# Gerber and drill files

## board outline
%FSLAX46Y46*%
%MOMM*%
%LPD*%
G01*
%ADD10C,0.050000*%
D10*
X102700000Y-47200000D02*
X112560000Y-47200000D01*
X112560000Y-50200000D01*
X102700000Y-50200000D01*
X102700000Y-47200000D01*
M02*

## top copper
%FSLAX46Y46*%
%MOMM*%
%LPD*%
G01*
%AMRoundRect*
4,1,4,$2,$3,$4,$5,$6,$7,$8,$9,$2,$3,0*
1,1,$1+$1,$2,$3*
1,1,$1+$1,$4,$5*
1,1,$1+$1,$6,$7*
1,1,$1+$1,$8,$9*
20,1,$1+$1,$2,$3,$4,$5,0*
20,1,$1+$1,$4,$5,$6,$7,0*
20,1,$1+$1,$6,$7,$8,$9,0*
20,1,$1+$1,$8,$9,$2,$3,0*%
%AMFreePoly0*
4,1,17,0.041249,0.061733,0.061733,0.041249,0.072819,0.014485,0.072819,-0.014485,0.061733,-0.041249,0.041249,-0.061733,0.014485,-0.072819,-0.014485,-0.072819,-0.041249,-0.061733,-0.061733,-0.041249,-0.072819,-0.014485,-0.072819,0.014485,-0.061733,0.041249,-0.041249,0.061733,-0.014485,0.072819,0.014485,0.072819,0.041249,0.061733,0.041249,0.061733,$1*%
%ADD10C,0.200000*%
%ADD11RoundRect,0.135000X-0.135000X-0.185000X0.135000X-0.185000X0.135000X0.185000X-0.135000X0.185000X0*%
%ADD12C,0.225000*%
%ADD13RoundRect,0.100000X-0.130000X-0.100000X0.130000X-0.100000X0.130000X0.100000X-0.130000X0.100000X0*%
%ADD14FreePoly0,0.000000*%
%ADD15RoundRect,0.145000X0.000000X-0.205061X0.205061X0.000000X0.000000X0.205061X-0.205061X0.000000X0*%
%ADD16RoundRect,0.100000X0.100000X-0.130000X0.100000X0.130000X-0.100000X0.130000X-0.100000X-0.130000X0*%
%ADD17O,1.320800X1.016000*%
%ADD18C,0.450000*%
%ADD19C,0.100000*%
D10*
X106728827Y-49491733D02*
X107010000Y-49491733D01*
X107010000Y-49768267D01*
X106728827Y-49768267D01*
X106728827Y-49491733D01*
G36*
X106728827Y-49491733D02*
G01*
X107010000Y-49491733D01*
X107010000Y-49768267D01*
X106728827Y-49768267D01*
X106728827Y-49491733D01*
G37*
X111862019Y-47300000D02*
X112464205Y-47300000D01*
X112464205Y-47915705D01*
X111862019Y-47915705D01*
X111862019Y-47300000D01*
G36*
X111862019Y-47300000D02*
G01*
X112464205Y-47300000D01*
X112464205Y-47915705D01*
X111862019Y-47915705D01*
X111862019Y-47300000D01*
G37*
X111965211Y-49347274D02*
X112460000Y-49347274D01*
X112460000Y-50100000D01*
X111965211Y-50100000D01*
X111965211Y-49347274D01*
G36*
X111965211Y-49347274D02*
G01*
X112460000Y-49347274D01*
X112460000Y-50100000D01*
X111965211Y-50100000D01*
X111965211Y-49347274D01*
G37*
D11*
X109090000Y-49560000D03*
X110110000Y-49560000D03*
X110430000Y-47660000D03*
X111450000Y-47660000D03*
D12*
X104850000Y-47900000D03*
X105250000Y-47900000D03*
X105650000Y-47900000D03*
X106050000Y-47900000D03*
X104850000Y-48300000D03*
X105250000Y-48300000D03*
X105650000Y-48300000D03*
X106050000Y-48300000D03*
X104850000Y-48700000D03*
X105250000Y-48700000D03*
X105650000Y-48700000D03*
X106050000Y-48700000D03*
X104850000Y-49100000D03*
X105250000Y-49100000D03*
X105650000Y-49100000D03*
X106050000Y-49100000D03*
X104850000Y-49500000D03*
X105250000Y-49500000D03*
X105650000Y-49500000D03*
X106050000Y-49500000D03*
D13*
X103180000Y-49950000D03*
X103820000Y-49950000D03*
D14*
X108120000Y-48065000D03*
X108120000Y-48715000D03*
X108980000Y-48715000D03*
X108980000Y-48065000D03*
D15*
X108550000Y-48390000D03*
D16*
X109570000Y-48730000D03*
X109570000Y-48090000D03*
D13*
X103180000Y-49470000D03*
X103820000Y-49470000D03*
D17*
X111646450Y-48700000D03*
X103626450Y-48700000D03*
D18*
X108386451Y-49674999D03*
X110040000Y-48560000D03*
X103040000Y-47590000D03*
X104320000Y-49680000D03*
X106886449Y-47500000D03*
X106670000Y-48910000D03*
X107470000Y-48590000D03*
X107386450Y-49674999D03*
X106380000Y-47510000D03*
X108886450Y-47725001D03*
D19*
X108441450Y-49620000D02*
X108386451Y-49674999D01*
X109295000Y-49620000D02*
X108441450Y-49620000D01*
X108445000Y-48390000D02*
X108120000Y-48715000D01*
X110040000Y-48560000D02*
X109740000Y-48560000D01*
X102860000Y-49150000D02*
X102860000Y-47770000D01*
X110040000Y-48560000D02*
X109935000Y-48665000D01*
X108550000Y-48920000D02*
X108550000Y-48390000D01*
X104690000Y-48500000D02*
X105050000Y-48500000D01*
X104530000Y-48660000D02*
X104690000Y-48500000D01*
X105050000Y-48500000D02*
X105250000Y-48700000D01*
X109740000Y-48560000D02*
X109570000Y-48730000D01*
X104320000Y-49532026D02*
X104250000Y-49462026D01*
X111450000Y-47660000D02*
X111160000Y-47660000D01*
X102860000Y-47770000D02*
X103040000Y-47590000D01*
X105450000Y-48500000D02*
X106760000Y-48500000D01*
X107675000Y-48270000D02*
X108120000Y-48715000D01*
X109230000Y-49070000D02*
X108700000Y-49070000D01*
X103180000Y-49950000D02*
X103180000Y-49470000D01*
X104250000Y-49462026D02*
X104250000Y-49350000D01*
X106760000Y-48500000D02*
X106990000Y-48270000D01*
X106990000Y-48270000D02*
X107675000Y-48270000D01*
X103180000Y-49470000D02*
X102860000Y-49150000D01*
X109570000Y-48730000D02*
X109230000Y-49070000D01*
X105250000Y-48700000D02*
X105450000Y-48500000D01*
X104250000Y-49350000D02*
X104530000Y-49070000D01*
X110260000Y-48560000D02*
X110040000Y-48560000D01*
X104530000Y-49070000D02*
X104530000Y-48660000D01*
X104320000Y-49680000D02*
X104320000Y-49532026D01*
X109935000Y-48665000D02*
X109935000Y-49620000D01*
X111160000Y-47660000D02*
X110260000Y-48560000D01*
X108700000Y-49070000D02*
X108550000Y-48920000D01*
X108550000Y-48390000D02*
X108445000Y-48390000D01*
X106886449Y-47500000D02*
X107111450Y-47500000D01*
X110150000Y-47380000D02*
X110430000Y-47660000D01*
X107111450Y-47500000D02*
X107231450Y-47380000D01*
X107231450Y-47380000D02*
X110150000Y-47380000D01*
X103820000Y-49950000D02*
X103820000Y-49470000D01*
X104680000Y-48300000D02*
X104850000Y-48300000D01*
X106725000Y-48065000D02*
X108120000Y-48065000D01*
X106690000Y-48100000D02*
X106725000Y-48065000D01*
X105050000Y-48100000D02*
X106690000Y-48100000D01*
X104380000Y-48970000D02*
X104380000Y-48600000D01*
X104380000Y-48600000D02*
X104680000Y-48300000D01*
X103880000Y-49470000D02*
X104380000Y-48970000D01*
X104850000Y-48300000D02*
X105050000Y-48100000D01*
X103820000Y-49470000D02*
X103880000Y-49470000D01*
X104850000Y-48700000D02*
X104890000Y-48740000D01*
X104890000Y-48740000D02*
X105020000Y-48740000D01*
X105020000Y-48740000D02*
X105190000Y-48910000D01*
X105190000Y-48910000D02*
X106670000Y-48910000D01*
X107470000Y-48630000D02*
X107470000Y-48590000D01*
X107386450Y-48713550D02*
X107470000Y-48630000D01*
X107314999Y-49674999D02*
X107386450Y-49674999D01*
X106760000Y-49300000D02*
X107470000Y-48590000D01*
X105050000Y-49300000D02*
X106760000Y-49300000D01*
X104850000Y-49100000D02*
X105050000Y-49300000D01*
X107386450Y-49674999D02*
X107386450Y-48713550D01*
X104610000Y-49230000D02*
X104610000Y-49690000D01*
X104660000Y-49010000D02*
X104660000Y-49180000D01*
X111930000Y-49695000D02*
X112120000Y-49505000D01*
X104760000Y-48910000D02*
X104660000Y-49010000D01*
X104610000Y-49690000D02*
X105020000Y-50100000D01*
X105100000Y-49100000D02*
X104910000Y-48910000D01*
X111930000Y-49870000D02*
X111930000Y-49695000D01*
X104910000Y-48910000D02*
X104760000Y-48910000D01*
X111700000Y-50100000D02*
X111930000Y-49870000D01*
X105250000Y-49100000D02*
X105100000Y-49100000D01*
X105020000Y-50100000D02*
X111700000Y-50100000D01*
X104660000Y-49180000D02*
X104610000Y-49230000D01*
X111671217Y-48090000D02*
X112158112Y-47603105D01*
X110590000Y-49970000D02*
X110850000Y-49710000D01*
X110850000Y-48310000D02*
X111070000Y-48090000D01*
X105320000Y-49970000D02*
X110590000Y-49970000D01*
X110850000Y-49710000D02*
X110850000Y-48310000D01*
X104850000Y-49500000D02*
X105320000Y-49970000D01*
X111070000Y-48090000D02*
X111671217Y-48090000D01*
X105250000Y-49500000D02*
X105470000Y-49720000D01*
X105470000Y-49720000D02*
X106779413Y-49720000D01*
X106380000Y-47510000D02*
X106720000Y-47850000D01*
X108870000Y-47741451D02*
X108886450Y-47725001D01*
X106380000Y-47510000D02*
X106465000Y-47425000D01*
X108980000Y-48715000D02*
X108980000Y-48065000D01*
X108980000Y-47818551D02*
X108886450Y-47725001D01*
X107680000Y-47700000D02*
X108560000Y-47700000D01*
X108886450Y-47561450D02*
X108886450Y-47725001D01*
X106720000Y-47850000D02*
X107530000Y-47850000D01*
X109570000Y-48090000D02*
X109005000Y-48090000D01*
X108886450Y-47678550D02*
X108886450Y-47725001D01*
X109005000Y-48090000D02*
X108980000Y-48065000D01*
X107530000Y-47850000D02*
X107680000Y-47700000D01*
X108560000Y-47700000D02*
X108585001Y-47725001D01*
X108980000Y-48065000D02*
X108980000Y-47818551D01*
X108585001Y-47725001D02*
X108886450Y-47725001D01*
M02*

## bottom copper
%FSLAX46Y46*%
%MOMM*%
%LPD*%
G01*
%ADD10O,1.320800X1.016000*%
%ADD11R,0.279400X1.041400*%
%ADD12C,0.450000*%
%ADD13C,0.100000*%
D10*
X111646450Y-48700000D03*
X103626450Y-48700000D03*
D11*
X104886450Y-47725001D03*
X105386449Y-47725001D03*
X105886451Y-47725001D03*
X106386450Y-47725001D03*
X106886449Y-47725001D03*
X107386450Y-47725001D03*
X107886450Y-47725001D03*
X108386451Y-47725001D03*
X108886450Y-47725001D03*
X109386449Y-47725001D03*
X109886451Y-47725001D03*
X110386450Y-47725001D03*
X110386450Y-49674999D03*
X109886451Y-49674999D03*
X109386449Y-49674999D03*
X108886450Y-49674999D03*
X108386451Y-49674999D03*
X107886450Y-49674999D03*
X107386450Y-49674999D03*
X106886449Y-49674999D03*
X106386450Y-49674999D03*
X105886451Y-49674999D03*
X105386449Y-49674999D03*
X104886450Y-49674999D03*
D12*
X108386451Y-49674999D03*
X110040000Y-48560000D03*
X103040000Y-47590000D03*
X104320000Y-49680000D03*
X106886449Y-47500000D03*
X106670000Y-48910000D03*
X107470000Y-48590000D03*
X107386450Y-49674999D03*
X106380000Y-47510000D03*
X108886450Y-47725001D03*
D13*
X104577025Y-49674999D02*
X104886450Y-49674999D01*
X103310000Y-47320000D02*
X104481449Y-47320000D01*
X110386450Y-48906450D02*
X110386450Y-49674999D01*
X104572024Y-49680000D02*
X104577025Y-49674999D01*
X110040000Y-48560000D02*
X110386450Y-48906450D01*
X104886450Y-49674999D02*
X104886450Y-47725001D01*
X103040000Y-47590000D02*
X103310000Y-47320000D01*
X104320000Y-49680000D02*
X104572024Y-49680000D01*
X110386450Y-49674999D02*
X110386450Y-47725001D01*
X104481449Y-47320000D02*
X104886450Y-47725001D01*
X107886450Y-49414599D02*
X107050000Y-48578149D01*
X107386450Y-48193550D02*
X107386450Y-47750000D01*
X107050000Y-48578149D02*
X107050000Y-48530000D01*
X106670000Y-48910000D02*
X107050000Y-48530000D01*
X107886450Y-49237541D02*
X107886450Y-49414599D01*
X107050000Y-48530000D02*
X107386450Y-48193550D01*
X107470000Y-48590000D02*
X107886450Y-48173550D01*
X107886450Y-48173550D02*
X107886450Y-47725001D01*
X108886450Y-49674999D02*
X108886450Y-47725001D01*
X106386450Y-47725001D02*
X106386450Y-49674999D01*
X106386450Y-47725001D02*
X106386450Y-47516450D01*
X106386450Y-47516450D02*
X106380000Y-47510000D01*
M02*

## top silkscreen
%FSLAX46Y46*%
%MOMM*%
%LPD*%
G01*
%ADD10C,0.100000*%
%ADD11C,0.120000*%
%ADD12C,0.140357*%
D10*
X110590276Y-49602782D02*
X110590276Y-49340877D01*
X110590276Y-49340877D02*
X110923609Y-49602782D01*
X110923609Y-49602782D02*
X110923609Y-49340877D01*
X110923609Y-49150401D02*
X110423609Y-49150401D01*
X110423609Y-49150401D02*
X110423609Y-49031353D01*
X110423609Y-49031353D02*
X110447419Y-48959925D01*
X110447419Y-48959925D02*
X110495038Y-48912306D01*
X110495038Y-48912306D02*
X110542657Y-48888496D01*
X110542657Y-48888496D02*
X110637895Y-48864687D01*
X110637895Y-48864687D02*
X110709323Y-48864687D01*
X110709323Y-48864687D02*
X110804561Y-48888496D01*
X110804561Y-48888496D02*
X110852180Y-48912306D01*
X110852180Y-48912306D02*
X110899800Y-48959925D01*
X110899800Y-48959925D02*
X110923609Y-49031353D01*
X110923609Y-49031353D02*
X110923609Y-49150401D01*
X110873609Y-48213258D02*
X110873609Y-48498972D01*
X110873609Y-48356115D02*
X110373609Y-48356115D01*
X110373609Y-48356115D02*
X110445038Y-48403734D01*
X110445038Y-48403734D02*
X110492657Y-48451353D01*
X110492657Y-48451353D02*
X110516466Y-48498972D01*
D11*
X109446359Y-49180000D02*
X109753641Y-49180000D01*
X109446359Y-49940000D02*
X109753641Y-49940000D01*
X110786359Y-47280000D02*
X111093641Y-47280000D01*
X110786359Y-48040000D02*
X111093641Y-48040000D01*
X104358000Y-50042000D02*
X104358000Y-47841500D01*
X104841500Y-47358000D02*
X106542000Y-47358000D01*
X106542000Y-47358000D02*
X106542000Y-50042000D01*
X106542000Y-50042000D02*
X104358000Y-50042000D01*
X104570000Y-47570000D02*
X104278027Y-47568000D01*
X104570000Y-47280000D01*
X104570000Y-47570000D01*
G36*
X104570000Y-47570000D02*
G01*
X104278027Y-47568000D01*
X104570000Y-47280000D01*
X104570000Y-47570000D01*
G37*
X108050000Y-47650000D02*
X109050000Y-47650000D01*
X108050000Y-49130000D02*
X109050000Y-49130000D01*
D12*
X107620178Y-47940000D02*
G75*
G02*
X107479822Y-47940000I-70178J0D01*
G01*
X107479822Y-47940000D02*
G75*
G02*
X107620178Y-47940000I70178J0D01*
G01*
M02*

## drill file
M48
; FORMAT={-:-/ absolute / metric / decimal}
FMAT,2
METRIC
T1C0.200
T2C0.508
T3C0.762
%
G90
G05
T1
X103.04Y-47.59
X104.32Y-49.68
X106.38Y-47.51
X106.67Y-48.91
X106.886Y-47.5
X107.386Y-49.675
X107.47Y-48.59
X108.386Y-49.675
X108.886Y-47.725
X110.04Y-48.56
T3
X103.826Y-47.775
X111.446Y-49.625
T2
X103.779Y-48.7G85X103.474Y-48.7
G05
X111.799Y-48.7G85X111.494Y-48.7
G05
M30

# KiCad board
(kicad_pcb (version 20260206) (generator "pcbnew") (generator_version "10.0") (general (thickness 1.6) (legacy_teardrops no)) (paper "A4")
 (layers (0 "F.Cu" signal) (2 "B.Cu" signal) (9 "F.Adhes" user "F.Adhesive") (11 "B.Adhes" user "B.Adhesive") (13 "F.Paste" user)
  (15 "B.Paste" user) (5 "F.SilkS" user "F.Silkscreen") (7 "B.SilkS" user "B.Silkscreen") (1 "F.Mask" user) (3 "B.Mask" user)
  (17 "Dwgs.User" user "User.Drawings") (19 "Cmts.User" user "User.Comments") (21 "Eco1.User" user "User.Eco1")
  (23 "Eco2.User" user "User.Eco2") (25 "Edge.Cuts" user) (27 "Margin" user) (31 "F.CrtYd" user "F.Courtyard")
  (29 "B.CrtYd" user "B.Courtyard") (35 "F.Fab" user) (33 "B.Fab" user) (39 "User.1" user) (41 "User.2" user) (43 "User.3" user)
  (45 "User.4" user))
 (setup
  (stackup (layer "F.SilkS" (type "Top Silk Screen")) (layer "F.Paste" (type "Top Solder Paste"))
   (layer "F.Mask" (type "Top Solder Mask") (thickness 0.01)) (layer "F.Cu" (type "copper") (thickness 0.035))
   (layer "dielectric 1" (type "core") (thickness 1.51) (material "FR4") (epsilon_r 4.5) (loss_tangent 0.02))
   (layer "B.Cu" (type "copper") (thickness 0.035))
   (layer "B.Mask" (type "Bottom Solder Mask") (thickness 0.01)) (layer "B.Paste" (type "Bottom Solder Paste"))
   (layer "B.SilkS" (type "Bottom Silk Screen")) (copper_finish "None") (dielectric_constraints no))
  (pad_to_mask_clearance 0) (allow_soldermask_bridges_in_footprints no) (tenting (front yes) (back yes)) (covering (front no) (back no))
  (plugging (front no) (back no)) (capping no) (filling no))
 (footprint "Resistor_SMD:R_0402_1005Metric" (layer "F.Cu") (at 109.6 49.56)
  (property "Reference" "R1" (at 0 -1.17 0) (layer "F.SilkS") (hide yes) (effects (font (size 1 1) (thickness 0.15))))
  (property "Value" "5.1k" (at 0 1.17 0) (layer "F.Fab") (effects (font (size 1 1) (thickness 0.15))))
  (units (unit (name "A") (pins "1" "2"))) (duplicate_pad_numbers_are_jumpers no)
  (fp_line (start -0.153641 -0.38) (end 0.153641 -0.38) (stroke (width 0.12) (type solid)) (layer "F.SilkS"))
  (fp_line (start -0.153641 0.38) (end 0.153641 0.38) (stroke (width 0.12) (type solid)) (layer "F.SilkS"))
  (pad "1" smd roundrect (at -0.51 0) (size 0.54 0.64) (layers "F.Cu" "F.Mask" "F.Paste") (roundrect_rratio 0.25) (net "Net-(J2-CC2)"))
  (pad "2" smd roundrect (at 0.51 0) (size 0.54 0.64) (layers "F.Cu" "F.Mask" "F.Paste") (roundrect_rratio 0.25) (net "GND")))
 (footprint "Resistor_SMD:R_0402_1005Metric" (layer "F.Cu") (at 110.94 47.66)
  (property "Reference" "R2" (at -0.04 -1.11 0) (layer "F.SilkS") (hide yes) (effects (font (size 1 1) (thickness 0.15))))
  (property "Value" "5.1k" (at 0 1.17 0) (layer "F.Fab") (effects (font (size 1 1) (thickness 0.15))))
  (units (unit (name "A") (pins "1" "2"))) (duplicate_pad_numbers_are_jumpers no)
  (fp_line (start -0.153641 -0.38) (end 0.153641 -0.38) (stroke (width 0.12) (type solid)) (layer "F.SilkS"))
  (fp_line (start -0.153641 0.38) (end 0.153641 0.38) (stroke (width 0.12) (type solid)) (layer "F.SilkS"))
  (pad "1" smd roundrect (at -0.51 0) (size 0.54 0.64) (layers "F.Cu" "F.Mask" "F.Paste") (roundrect_rratio 0.25) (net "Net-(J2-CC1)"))
  (pad "2" smd roundrect (at 0.51 0) (size 0.54 0.64) (layers "F.Cu" "F.Mask" "F.Paste") (roundrect_rratio 0.25) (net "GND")))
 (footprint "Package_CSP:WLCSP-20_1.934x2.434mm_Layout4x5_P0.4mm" (layer "F.Cu") (at 105.45 48.7)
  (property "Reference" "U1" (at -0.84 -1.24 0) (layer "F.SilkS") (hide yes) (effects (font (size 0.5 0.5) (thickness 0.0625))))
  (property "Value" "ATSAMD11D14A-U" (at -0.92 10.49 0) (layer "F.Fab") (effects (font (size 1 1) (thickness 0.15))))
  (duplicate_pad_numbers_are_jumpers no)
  (fp_line (start -1.092 1.342) (end -1.092 -0.8585) (stroke (width 0.12) (type solid)) (layer "F.SilkS"))
  (fp_line (start -0.6085 -1.342) (end 1.092 -1.342) (stroke (width 0.12) (type solid)) (layer "F.SilkS"))
  (fp_line (start 1.092 -1.342) (end 1.092 1.342) (stroke (width 0.12) (type solid)) (layer "F.SilkS"))
  (fp_line (start 1.092 1.342) (end -1.092 1.342) (stroke (width 0.12) (type solid)) (layer "F.SilkS"))
  (fp_poly (pts (xy -0.88 -1.13) (xy -1.171973 -1.132) (xy -0.88 -1.42)) (stroke (width 0.12) (type solid)) (fill yes) (layer "F.SilkS"))
  (pad "A1" smd circle (at -0.6 -0.8) (size 0.225 0.225) (layers "F.Cu" "F.Mask" "F.Paste") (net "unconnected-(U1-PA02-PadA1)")
   (solder_paste_margin_ratio 0.055556))
  (pad "A2" smd circle (at -0.2 -0.8) (size 0.225 0.225) (layers "F.Cu" "F.Mask" "F.Paste") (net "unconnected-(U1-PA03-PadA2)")
   (solder_paste_margin_ratio 0.055556))
  (pad "A3" smd circle (at 0.2 -0.8) (size 0.225 0.225) (layers "F.Cu" "F.Mask" "F.Paste") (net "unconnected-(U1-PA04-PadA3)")
   (solder_paste_margin_ratio 0.055556))
  (pad "A4" smd circle (at 0.6 -0.8) (size 0.225 0.225) (layers "F.Cu" "F.Mask" "F.Paste") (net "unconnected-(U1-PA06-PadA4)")
   (solder_paste_margin_ratio 0.055556))
  (pad "B1" smd circle (at -0.6 -0.4) (size 0.225 0.225) (layers "F.Cu" "F.Mask" "F.Paste") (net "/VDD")
   (solder_paste_margin_ratio 0.055556))
  (pad "B2" smd circle (at -0.2 -0.4) (size 0.225 0.225) (layers "F.Cu" "F.Mask" "F.Paste") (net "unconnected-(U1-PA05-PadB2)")
   (solder_paste_margin_ratio 0.055556))
  (pad "B3" smd circle (at 0.2 -0.4) (size 0.225 0.225) (layers "F.Cu" "F.Mask" "F.Paste") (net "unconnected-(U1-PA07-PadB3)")
   (solder_paste_margin_ratio 0.055556))
  (pad "B4" smd circle (at 0.6 -0.4) (size 0.225 0.225) (layers "F.Cu" "F.Mask" "F.Paste") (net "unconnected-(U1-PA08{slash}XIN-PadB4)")
   (solder_paste_margin_ratio 0.055556))
  (pad "C1" smd circle (at -0.6 0) (size 0.225 0.225) (layers "F.Cu" "F.Mask" "F.Paste") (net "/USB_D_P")
   (solder_paste_margin_ratio 0.055556))
  (pad "C2" smd circle (at -0.2 0) (size 0.225 0.225) (layers "F.Cu" "F.Mask" "F.Paste") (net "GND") (solder_paste_margin_ratio 0.055556))
  (pad "C3" smd circle (at 0.2 0) (size 0.225 0.225) (layers "F.Cu" "F.Mask" "F.Paste") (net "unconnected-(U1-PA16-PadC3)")
   (solder_paste_margin_ratio 0.055556))
  (pad "C4" smd circle (at 0.6 0) (size 0.225 0.225) (layers "F.Cu" "F.Mask" "F.Paste") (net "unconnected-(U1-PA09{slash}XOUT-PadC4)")
   (solder_paste_margin_ratio 0.055556))
  (pad "D1" smd circle (at -0.6 0.4) (size 0.225 0.225) (layers "F.Cu" "F.Mask" "F.Paste") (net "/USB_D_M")
   (solder_paste_margin_ratio 0.055556))
  (pad "D2" smd circle (at -0.2 0.4) (size 0.225 0.225) (layers "F.Cu" "F.Mask" "F.Paste") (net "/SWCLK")
   (solder_paste_margin_ratio 0.055556))
  (pad "D3" smd circle (at 0.2 0.4) (size 0.225 0.225) (layers "F.Cu" "F.Mask" "F.Paste") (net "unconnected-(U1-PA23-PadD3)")
   (solder_paste_margin_ratio 0.055556))
  (pad "D4" smd circle (at 0.6 0.4) (size 0.225 0.225) (layers "F.Cu" "F.Mask" "F.Paste") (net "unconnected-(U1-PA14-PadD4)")
   (solder_paste_margin_ratio 0.055556))
  (pad "E1" smd circle (at -0.6 0.8) (size 0.225 0.225) (layers "F.Cu" "F.Mask" "F.Paste") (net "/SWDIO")
   (solder_paste_margin_ratio 0.055556))
  (pad "E2" smd circle (at -0.2 0.8) (size 0.225 0.225) (layers "F.Cu" "F.Mask" "F.Paste") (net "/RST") (solder_paste_margin_ratio 0.055556))
  (pad "E3" smd circle (at 0.2 0.8) (size 0.225 0.225) (layers "F.Cu" "F.Mask" "F.Paste") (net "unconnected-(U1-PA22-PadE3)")
   (solder_paste_margin_ratio 0.055556))
  (pad "E4" smd circle (at 0.6 0.8) (size 0.225 0.225) (layers "F.Cu" "F.Mask" "F.Paste") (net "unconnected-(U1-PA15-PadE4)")
   (solder_paste_margin_ratio 0.055556)))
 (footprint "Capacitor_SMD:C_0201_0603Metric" (layer "F.Cu") (at 103.5 49.95)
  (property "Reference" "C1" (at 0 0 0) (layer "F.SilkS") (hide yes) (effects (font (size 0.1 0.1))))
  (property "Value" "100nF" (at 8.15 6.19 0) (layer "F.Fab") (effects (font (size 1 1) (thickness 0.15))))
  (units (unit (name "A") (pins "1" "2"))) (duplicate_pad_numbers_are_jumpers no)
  (pad "" smd roundrect (at -0.345 0) (size 0.318 0.36) (layers "F.Paste") (roundrect_rratio 0.25))
  (pad "" smd roundrect (at 0.345 0) (size 0.318 0.36) (layers "F.Paste") (roundrect_rratio 0.25))
  (pad "1" smd roundrect (at -0.32 0) (size 0.46 0.4) (layers "F.Cu" "F.Mask") (roundrect_rratio 0.25) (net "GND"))
  (pad "2" smd roundrect (at 0.32 0) (size 0.46 0.4) (layers "F.Cu" "F.Mask") (roundrect_rratio 0.25) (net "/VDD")))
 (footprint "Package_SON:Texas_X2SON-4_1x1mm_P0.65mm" (layer "F.Cu") (at 108.55 48.39)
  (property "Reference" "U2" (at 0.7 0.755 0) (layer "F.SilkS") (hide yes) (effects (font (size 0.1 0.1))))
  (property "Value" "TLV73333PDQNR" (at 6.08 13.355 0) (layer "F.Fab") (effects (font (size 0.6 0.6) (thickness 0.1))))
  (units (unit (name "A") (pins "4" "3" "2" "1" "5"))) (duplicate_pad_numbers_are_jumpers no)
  (fp_line (start -0.5 -0.74) (end 0.5 -0.74) (stroke (width 0.12) (type solid)) (layer "F.SilkS"))
  (fp_line (start -0.5 0.74) (end 0.5 0.74) (stroke (width 0.12) (type solid)) (layer "F.SilkS"))
  (fp_circle (center -1 -0.45) (end -0.86 -0.46) (stroke (width 0) (type solid)) (fill yes) (layer "F.SilkS"))
  (pad "" smd custom (at -0.43 -0.325) (size 0.148492 0.148492) (layers "F.Mask") (thermal_bridge_angle 90)
   (options (clearance outline) (anchor circle)) (primitives))
  (pad "" smd custom (at -0.43 -0.325) (size 0.148492 0.148492) (layers "F.Paste") (thermal_bridge_angle 90)
   (options (clearance outline) (anchor circle)) (primitives))
  (pad "" smd custom (at -0.43 0.325) (size 0.148492 0.148492) (layers "F.Mask") (thermal_bridge_angle 90)
   (options (clearance outline) (anchor circle)) (primitives))
  (pad "" smd custom (at -0.43 0.325) (size 0.148492 0.148492) (layers "F.Paste") (thermal_bridge_angle 90)
   (options (clearance outline) (anchor circle)) (primitives))
  (pad "" smd custom (at 0.43 -0.325) (size 0.148492 0.148492) (layers "F.Mask") (thermal_bridge_angle 90)
   (options (clearance outline) (anchor circle)) (primitives))
  (pad "" smd custom (at 0.43 -0.325) (size 0.148492 0.148492) (layers "F.Paste") (thermal_bridge_angle 90)
   (options (clearance outline) (anchor circle)) (primitives))
  (pad "" smd custom (at 0.43 0.325) (size 0.148492 0.148492) (layers "F.Mask") (thermal_bridge_angle 90)
   (options (clearance outline) (anchor circle)) (primitives))
  (pad "" smd custom (at 0.43 0.325) (size 0.148492 0.148492) (layers "F.Paste") (thermal_bridge_angle 90)
   (options (clearance outline) (anchor circle)) (primitives))
  (pad "1" smd custom (at -0.43 -0.325) (size 0.148492 0.148492) (layers "F.Cu") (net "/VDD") (zone_connect 2) (thermal_bridge_angle 90)
   (options (clearance outline) (anchor circle)) (primitives))
  (pad "2" smd custom (at -0.43 0.325) (size 0.148492 0.148492) (layers "F.Cu") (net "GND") (zone_connect 2) (thermal_bridge_angle 90)
   (options (clearance outline) (anchor circle)) (primitives))
  (pad "3" smd custom (at 0.43 0.325) (size 0.148492 0.148492) (layers "F.Cu") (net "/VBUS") (zone_connect 2) (thermal_bridge_angle 90)
   (options (clearance outline) (anchor circle)) (primitives))
  (pad "4" smd custom (at 0.43 -0.325) (size 0.148492 0.148492) (layers "F.Cu") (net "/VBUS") (zone_connect 2) (thermal_bridge_angle 90)
   (options (clearance outline) (anchor circle)) (primitives))
  (pad "5" smd roundrect (at 0 0 45) (size 0.58 0.58) (layers "F.Cu" "F.Mask" "F.Paste") (roundrect_rratio 0.25) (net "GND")
   (solder_mask_margin -0.05) (solder_paste_margin -0.065) (solder_paste_margin_ratio -0.00000001)))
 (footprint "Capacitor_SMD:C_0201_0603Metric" (layer "F.Cu") (at 109.57 48.41 90)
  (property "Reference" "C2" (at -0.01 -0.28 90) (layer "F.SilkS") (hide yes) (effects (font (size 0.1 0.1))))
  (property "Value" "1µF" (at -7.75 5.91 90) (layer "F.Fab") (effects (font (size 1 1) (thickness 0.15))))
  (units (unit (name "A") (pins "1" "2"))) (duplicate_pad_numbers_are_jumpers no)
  (pad "" smd roundrect (at -0.345 0 90) (size 0.318 0.36) (layers "F.Paste") (roundrect_rratio 0.25))
  (pad "" smd roundrect (at 0.345 0 90) (size 0.318 0.36) (layers "F.Paste") (roundrect_rratio 0.25))
  (pad "1" smd roundrect (at -0.32 0 90) (size 0.46 0.4) (layers "F.Cu" "F.Mask") (roundrect_rratio 0.25) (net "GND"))
  (pad "2" smd roundrect (at 0.32 0 90) (size 0.46 0.4) (layers "F.Cu" "F.Mask") (roundrect_rratio 0.25) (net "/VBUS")))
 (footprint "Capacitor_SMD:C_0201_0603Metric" (layer "F.Cu") (at 103.5 49.47)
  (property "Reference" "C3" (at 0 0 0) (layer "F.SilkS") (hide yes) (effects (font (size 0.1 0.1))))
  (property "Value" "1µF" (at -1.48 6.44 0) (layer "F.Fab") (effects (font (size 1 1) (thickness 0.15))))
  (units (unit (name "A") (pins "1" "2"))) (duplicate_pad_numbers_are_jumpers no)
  (pad "" smd roundrect (at -0.345 0) (size 0.318 0.36) (layers "F.Paste") (roundrect_rratio 0.25))
  (pad "" smd roundrect (at 0.345 0) (size 0.318 0.36) (layers "F.Paste") (roundrect_rratio 0.25))
  (pad "1" smd roundrect (at -0.32 0) (size 0.46 0.4) (layers "F.Cu" "F.Mask") (roundrect_rratio 0.25) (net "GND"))
  (pad "2" smd roundrect (at 0.32 0) (size 0.46 0.4) (layers "F.Cu" "F.Mask") (roundrect_rratio 0.25) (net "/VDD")))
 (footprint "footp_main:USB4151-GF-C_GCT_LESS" (layer "B.Cu") (at 107.63645 48.7 180)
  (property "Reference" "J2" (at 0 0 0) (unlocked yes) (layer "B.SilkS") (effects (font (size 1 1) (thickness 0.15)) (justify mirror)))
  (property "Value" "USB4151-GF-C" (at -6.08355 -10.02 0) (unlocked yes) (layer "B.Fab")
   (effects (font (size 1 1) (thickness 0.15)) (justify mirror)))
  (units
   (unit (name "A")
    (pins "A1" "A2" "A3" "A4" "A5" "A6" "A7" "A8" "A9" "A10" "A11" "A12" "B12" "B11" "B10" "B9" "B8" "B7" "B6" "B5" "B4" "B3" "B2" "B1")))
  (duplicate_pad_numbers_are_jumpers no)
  (pad "" np_thru_hole oval (at -4.01 0 180) (size 1.3208 1.016) (drill oval 0.8128 0.508) (layers "*.Cu" "*.Mask"))
  (pad "" np_thru_hole circle (at -3.81 -0.925 180) (size 0.762 0.762) (drill 0.762) (layers))
  (pad "" np_thru_hole circle (at 3.81 0.925 180) (size 0.762 0.762) (drill 0.762) (layers))
  (pad "" np_thru_hole oval (at 4.01 0 180) (size 1.3208 1.016) (drill oval 0.8128 0.508) (layers "*.Cu" "*.Mask"))
  (pad "A1" smd rect (at 2.75 0.974999 180) (size 0.2794 1.0414) (layers "B.Cu" "B.Mask" "B.Paste") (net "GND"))
  (pad "A2" smd rect (at 2.250001 0.974999 180) (size 0.2794 1.0414) (layers "B.Cu" "B.Mask" "B.Paste")
   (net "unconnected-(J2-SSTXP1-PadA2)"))
  (pad "A3" smd rect (at 1.749999 0.974999 180) (size 0.2794 1.0414) (layers "B.Cu" "B.Mask" "B.Paste")
   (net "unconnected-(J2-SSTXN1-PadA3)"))
  (pad "A4" smd rect (at 1.25 0.974999 180) (size 0.2794 1.0414) (layers "B.Cu" "B.Mask" "B.Paste") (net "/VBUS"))
  (pad "A5" smd rect (at 0.750001 0.974999 180) (size 0.2794 1.0414) (layers "B.Cu" "B.Mask" "B.Paste") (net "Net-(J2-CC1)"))
  (pad "A6" smd rect (at 0.25 0.974999 180) (size 0.2794 1.0414) (layers "B.Cu" "B.Mask" "B.Paste") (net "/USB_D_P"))
  (pad "A7" smd rect (at -0.25 0.974999 180) (size 0.2794 1.0414) (layers "B.Cu" "B.Mask" "B.Paste") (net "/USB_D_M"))
  (pad "A8" smd rect (at -0.750001 0.974999 180) (size 0.2794 1.0414) (layers "B.Cu" "B.Mask" "B.Paste") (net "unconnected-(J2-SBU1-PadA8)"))
  (pad "A9" smd rect (at -1.25 0.974999 180) (size 0.2794 1.0414) (layers "B.Cu" "B.Mask" "B.Paste") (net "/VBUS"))
  (pad "A10" smd rect (at -1.749999 0.974999 180) (size 0.2794 1.0414) (layers "B.Cu" "B.Mask" "B.Paste")
   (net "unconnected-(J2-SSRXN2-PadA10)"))
  (pad "A11" smd rect (at -2.250001 0.974999 180) (size 0.2794 1.0414) (layers "B.Cu" "B.Mask" "B.Paste")
   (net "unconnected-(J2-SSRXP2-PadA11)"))
  (pad "A12" smd rect (at -2.75 0.974999 180) (size 0.2794 1.0414) (layers "B.Cu" "B.Mask" "B.Paste") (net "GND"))
  (pad "B1" smd rect (at -2.75 -0.974999 180) (size 0.2794 1.0414) (layers "B.Cu" "B.Mask" "B.Paste") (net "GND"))
  (pad "B2" smd rect (at -2.250001 -0.974999 180) (size 0.2794 1.0414) (layers "B.Cu" "B.Mask" "B.Paste")
   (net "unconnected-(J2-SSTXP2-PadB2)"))
  (pad "B3" smd rect (at -1.749999 -0.974999 180) (size 0.2794 1.0414) (layers "B.Cu" "B.Mask" "B.Paste")
   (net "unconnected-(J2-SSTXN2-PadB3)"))
  (pad "B4" smd rect (at -1.25 -0.974999 180) (size 0.2794 1.0414) (layers "B.Cu" "B.Mask" "B.Paste") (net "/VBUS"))
  (pad "B5" smd rect (at -0.750001 -0.974999 180) (size 0.2794 1.0414) (layers "B.Cu" "B.Mask" "B.Paste") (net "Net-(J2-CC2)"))
  (pad "B6" smd rect (at -0.25 -0.974999 180) (size 0.2794 1.0414) (layers "B.Cu" "B.Mask" "B.Paste") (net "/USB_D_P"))
  (pad "B7" smd rect (at 0.25 -0.974999 180) (size 0.2794 1.0414) (layers "B.Cu" "B.Mask" "B.Paste") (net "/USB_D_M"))
  (pad "B8" smd rect (at 0.750001 -0.974999 180) (size 0.2794 1.0414) (layers "B.Cu" "B.Mask" "B.Paste") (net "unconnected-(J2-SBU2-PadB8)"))
  (pad "B9" smd rect (at 1.25 -0.974999 180) (size 0.2794 1.0414) (layers "B.Cu" "B.Mask" "B.Paste") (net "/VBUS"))
  (pad "B10" smd rect (at 1.749999 -0.974999 180) (size 0.2794 1.0414) (layers "B.Cu" "B.Mask" "B.Paste")
   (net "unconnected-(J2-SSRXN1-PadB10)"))
  (pad "B11" smd rect (at 2.250001 -0.974999 180) (size 0.2794 1.0414) (layers "B.Cu" "B.Mask" "B.Paste")
   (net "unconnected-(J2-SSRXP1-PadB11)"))
  (pad "B12" smd rect (at 2.75 -0.974999 180) (size 0.2794 1.0414) (layers "B.Cu" "B.Mask" "B.Paste") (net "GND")))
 (gr_rect (start 106.728827 49.491733) (end 107.01 49.768267) (stroke (width 0.2) (type solid)) (fill yes) (layer "F.Cu") (net "/RST"))
 (gr_rect (start 111.862019 47.3) (end 112.464205 47.915705) (stroke (width 0.2) (type solid)) (fill yes) (layer "F.Cu") (net "/SWDIO"))
 (gr_rect (start 111.965211 49.347274) (end 112.46 50.1) (stroke (width 0.2) (type solid)) (fill yes) (layer "F.Cu") (net "/SWCLK"))
 (gr_rect (start 102.7 47.2) (end 112.56 50.2) (stroke (width 0.05) (type default)) (fill no) (layer "Edge.Cuts"))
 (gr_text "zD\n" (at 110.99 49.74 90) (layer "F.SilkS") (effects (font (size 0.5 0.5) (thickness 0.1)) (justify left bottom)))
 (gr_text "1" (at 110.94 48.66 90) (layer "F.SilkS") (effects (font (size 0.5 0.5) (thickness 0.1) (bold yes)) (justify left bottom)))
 (segment (start 108.44145 49.62) (end 108.386451 49.674999) (width 0.1) (layer "F.Cu") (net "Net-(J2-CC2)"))
 (segment (start 109.295 49.62) (end 108.44145 49.62) (width 0.1) (layer "F.Cu") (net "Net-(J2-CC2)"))
 (via (at 108.386451 49.674999) (size 0.45) (drill 0.2) (layers "F.Cu" "B.Cu") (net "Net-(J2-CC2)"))
 (segment (start 108.445 48.39) (end 108.12 48.715) (width 0.1) (layer "F.Cu") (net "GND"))
 (segment (start 110.04 48.56) (end 109.74 48.56) (width 0.1) (layer "F.Cu") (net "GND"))
 (segment (start 102.86 49.15) (end 102.86 47.77) (width 0.1) (layer "F.Cu") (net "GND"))
 (segment (start 110.04 48.56) (end 109.935 48.665) (width 0.1) (layer "F.Cu") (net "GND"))
 (segment (start 108.55 48.92) (end 108.55 48.39) (width 0.1) (layer "F.Cu") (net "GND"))
 (segment (start 104.69 48.5) (end 105.05 48.5) (width 0.1) (layer "F.Cu") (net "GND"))
 (segment (start 104.53 48.66) (end 104.69 48.5) (width 0.1) (layer "F.Cu") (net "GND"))
 (segment (start 105.05 48.5) (end 105.25 48.7) (width 0.1) (layer "F.Cu") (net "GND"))
 (segment (start 109.74 48.56) (end 109.57 48.73) (width 0.1) (layer "F.Cu") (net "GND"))
 (segment (start 104.32 49.532026) (end 104.25 49.462026) (width 0.1) (layer "F.Cu") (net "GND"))
 (segment (start 111.45 47.66) (end 111.16 47.66) (width 0.1) (layer "F.Cu") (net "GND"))
 (segment (start 102.86 47.77) (end 103.04 47.59) (width 0.1) (layer "F.Cu") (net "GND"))
 (segment (start 105.45 48.5) (end 106.76 48.5) (width 0.1) (layer "F.Cu") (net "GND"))
 (segment (start 107.675 48.27) (end 108.12 48.715) (width 0.1) (layer "F.Cu") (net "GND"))
 (segment (start 109.23 49.07) (end 108.7 49.07) (width 0.1) (layer "F.Cu") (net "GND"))
 (segment (start 103.18 49.95) (end 103.18 49.47) (width 0.1) (layer "F.Cu") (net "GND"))
 (segment (start 104.25 49.462026) (end 104.25 49.35) (width 0.1) (layer "F.Cu") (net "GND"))
 (segment (start 106.76 48.5) (end 106.99 48.27) (width 0.1) (layer "F.Cu") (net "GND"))
 (segment (start 106.99 48.27) (end 107.675 48.27) (width 0.1) (layer "F.Cu") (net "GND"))
 (segment (start 103.18 49.47) (end 102.86 49.15) (width 0.1) (layer "F.Cu") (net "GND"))
 (segment (start 109.57 48.73) (end 109.23 49.07) (width 0.1) (layer "F.Cu") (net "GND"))
 (segment (start 105.25 48.7) (end 105.45 48.5) (width 0.1) (layer "F.Cu") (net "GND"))
 (segment (start 104.25 49.35) (end 104.53 49.07) (width 0.1) (layer "F.Cu") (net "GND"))
 (segment (start 110.26 48.56) (end 110.04 48.56) (width 0.1) (layer "F.Cu") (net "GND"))
 (segment (start 104.53 49.07) (end 104.53 48.66) (width 0.1) (layer "F.Cu") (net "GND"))
 (segment (start 104.32 49.68) (end 104.32 49.532026) (width 0.1) (layer "F.Cu") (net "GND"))
 (segment (start 109.935 48.665) (end 109.935 49.62) (width 0.1) (layer "F.Cu") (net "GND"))
 (segment (start 111.16 47.66) (end 110.26 48.56) (width 0.1) (layer "F.Cu") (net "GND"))
 (segment (start 108.7 49.07) (end 108.55 48.92) (width 0.1) (layer "F.Cu") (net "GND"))
 (segment (start 108.55 48.39) (end 108.445 48.39) (width 0.1) (layer "F.Cu") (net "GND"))
 (via (at 110.04 48.56) (size 0.45) (drill 0.2) (layers "F.Cu" "B.Cu") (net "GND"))
 (via (at 103.04 47.59) (size 0.45) (drill 0.2) (layers "F.Cu" "B.Cu") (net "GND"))
 (via (at 104.32 49.68) (size 0.45) (drill 0.2) (layers "F.Cu" "B.Cu") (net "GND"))
 (segment (start 104.577025 49.674999) (end 104.88645 49.674999) (width 0.1) (layer "B.Cu") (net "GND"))
 (segment (start 103.31 47.32) (end 104.481449 47.32) (width 0.1) (layer "B.Cu") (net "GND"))
 (segment (start 110.38645 48.90645) (end 110.38645 49.674999) (width 0.1) (layer "B.Cu") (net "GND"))
 (segment (start 104.572024 49.68) (end 104.577025 49.674999) (width 0.1) (layer "B.Cu") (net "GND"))
 (segment (start 110.04 48.56) (end 110.38645 48.90645) (width 0.1) (layer "B.Cu") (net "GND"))
 (segment (start 104.88645 49.674999) (end 104.88645 47.725001) (width 0.1) (layer "B.Cu") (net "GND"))
 (segment (start 103.04 47.59) (end 103.31 47.32) (width 0.1) (layer "B.Cu") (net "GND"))
 (segment (start 104.32 49.68) (end 104.572024 49.68) (width 0.1) (layer "B.Cu") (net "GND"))
 (segment (start 110.38645 49.674999) (end 110.38645 47.725001) (width 0.1) (layer "B.Cu") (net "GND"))
 (segment (start 104.481449 47.32) (end 104.88645 47.725001) (width 0.1) (layer "B.Cu") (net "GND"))
 (segment (start 106.886449 47.5) (end 107.11145 47.5) (width 0.1) (layer "F.Cu") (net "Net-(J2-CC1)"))
 (segment (start 110.15 47.38) (end 110.43 47.66) (width 0.1) (layer "F.Cu") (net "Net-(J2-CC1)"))
 (segment (start 107.11145 47.5) (end 107.23145 47.38) (width 0.1) (layer "F.Cu") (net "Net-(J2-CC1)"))
 (segment (start 107.23145 47.38) (end 110.15 47.38) (width 0.1) (layer "F.Cu") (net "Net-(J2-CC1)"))
 (via (at 106.886449 47.5) (size 0.45) (drill 0.2) (layers "F.Cu" "B.Cu") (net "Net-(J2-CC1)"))
 (segment (start 103.82 49.95) (end 103.82 49.47) (width 0.1) (layer "F.Cu") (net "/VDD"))
 (segment (start 104.68 48.3) (end 104.85 48.3) (width 0.1) (layer "F.Cu") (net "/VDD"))
 (segment (start 106.725 48.065) (end 108.12 48.065) (width 0.1) (layer "F.Cu") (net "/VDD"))
 (segment (start 106.69 48.1) (end 106.725 48.065) (width 0.1) (layer "F.Cu") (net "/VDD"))
 (segment (start 105.05 48.1) (end 106.69 48.1) (width 0.1) (layer "F.Cu") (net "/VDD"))
 (segment (start 104.38 48.97) (end 104.38 48.6) (width 0.1) (layer "F.Cu") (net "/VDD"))
 (segment (start 104.38 48.6) (end 104.68 48.3) (width 0.1) (layer "F.Cu") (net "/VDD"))
 (segment (start 103.88 49.47) (end 104.38 48.97) (width 0.1) (layer "F.Cu") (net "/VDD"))
 (segment (start 104.85 48.3) (end 105.05 48.1) (width 0.1) (layer "F.Cu") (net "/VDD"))
 (segment (start 103.82 49.47) (end 103.88 49.47) (width 0.1) (layer "F.Cu") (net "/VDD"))
 (segment (start 104.85 48.7) (end 104.89 48.74) (width 0.1) (layer "F.Cu") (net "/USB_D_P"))
 (segment (start 104.89 48.74) (end 105.02 48.74) (width 0.1) (layer "F.Cu") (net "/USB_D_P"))
 (segment (start 105.02 48.74) (end 105.19 48.91) (width 0.1) (layer "F.Cu") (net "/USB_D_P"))
 (segment (start 105.19 48.91) (end 106.67 48.91) (width 0.1) (layer "F.Cu") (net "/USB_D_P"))
 (via (at 106.67 48.91) (size 0.45) (drill 0.2) (layers "F.Cu" "B.Cu") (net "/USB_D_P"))
 (segment (start 107.88645 49.414599) (end 107.05 48.578149) (width 0.1) (layer "B.Cu") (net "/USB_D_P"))
 (segment (start 107.38645 48.19355) (end 107.38645 47.75) (width 0.1) (layer "B.Cu") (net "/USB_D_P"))
 (segment (start 107.05 48.578149) (end 107.05 48.53) (width 0.1) (layer "B.Cu") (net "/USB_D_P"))
 (segment (start 106.67 48.91) (end 107.05 48.53) (width 0.1) (layer "B.Cu") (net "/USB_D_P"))
 (segment (start 107.88645 49.237541) (end 107.88645 49.414599) (width 0.1) (layer "B.Cu") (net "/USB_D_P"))
 (segment (start 107.05 48.53) (end 107.38645 48.19355) (width 0.1) (layer "B.Cu") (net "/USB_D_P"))
 (segment (start 107.47 48.63) (end 107.47 48.59) (width 0.1) (layer "F.Cu") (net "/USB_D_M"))
 (segment (start 107.38645 48.71355) (end 107.47 48.63) (width 0.1) (layer "F.Cu") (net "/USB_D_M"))
 (segment (start 107.314999 49.674999) (end 107.38645 49.674999) (width 0.1) (layer "F.Cu") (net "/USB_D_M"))
 (segment (start 106.76 49.3) (end 107.47 48.59) (width 0.1) (layer "F.Cu") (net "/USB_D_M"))
 (segment (start 105.05 49.3) (end 106.76 49.3) (width 0.1) (layer "F.Cu") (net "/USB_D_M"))
 (segment (start 104.85 49.1) (end 105.05 49.3) (width 0.1) (layer "F.Cu") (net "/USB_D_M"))
 (segment (start 107.38645 49.674999) (end 107.38645 48.71355) (width 0.1) (layer "F.Cu") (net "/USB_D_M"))
 (via (at 107.47 48.59) (size 0.45) (drill 0.2) (layers "F.Cu" "B.Cu") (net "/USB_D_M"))
 (via (at 107.38645 49.674999) (size 0.45) (drill 0.2) (layers "F.Cu" "B.Cu") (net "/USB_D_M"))
 (segment (start 107.47 48.59) (end 107.88645 48.17355) (width 0.1) (layer "B.Cu") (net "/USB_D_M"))
 (segment (start 107.88645 48.17355) (end 107.88645 47.725001) (width 0.1) (layer "B.Cu") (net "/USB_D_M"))
 (segment (start 104.61 49.23) (end 104.61 49.69) (width 0.1) (layer "F.Cu") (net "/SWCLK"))
 (segment (start 104.66 49.01) (end 104.66 49.18) (width 0.1) (layer "F.Cu") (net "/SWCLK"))
 (segment (start 111.93 49.695) (end 112.12 49.505) (width 0.1) (layer "F.Cu") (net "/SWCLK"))
 (segment (start 104.76 48.91) (end 104.66 49.01) (width 0.1) (layer "F.Cu") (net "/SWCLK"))
 (segment (start 104.61 49.69) (end 105.02 50.1) (width 0.1) (layer "F.Cu") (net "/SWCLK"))
 (segment (start 105.1 49.1) (end 104.91 48.91) (width 0.1) (layer "F.Cu") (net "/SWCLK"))
 (segment (start 111.93 49.87) (end 111.93 49.695) (width 0.1) (layer "F.Cu") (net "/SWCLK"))
 (segment (start 104.91 48.91) (end 104.76 48.91) (width 0.1) (layer "F.Cu") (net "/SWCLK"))
 (segment (start 111.7 50.1) (end 111.93 49.87) (width 0.1) (layer "F.Cu") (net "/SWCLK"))
 (segment (start 105.25 49.1) (end 105.1 49.1) (width 0.1) (layer "F.Cu") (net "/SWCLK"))
 (segment (start 105.02 50.1) (end 111.7 50.1) (width 0.1) (layer "F.Cu") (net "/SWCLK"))
 (segment (start 104.66 49.18) (end 104.61 49.23) (width 0.1) (layer "F.Cu") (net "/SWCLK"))
 (segment (start 111.671217 48.09) (end 112.158112 47.603105) (width 0.1) (layer "F.Cu") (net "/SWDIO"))
 (segment (start 110.59 49.97) (end 110.85 49.71) (width 0.1) (layer "F.Cu") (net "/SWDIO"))
 (segment (start 110.85 48.31) (end 111.07 48.09) (width 0.1) (layer "F.Cu") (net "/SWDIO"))
 (segment (start 105.32 49.97) (end 110.59 49.97) (width 0.1) (layer "F.Cu") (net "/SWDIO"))
 (segment (start 110.85 49.71) (end 110.85 48.31) (width 0.1) (layer "F.Cu") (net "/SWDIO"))
 (segment (start 104.85 49.5) (end 105.32 49.97) (width 0.1) (layer "F.Cu") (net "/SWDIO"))
 (segment (start 111.07 48.09) (end 111.671217 48.09) (width 0.1) (layer "F.Cu") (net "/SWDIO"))
 (segment (start 105.25 49.5) (end 105.47 49.72) (width 0.1) (layer "F.Cu") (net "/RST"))
 (segment (start 105.47 49.72) (end 106.779413 49.72) (width 0.1) (layer "F.Cu") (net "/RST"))
 (segment (start 106.38 47.51) (end 106.72 47.85) (width 0.1) (layer "F.Cu") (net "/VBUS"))
 (segment (start 108.87 47.741451) (end 108.88645 47.725001) (width 0.1) (layer "F.Cu") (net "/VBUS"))
 (segment (start 106.38 47.51) (end 106.465 47.425) (width 0.1) (layer "F.Cu") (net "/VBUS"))
 (segment (start 108.98 48.715) (end 108.98 48.065) (width 0.1) (layer "F.Cu") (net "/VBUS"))
 (segment (start 108.98 47.818551) (end 108.88645 47.725001) (width 0.1) (layer "F.Cu") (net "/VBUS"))
 (segment (start 107.68 47.7) (end 108.56 47.7) (width 0.1) (layer "F.Cu") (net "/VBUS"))
 (segment (start 108.88645 47.56145) (end 108.88645 47.725001) (width 0.1) (layer "F.Cu") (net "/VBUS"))
 (segment (start 106.72 47.85) (end 107.53 47.85) (width 0.1) (layer "F.Cu") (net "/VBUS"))
 (segment (start 109.57 48.09) (end 109.005 48.09) (width 0.1) (layer "F.Cu") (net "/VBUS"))
 (segment (start 108.88645 47.67855) (end 108.88645 47.725001) (width 0.1) (layer "F.Cu") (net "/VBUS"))
 (segment (start 109.005 48.09) (end 108.98 48.065) (width 0.1) (layer "F.Cu") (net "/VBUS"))
 (segment (start 107.53 47.85) (end 107.68 47.7) (width 0.1) (layer "F.Cu") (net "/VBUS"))
 (segment (start 108.56 47.7) (end 108.585001 47.725001) (width 0.1) (layer "F.Cu") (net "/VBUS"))
 (segment (start 108.98 48.065) (end 108.98 47.818551) (width 0.1) (layer "F.Cu") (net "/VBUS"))
 (segment (start 108.585001 47.725001) (end 108.88645 47.725001) (width 0.1) (layer "F.Cu") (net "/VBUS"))
 (via (at 106.38 47.51) (size 0.45) (drill 0.2) (layers "F.Cu" "B.Cu") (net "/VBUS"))
 (via (at 108.88645 47.725001) (size 0.45) (drill 0.2) (layers "F.Cu" "B.Cu") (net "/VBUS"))
 (segment (start 108.88645 49.674999) (end 108.88645 47.725001) (width 0.1) (layer "B.Cu") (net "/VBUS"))
 (segment (start 106.38645 47.725001) (end 106.38645 49.674999) (width 0.1) (layer "B.Cu") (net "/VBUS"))
 (segment (start 106.38645 47.725001) (end 106.38645 47.51645) (width 0.1) (layer "B.Cu") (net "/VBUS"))
 (segment (start 106.38645 47.51645) (end 106.38 47.51) (width 0.1) (layer "B.Cu") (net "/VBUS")))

